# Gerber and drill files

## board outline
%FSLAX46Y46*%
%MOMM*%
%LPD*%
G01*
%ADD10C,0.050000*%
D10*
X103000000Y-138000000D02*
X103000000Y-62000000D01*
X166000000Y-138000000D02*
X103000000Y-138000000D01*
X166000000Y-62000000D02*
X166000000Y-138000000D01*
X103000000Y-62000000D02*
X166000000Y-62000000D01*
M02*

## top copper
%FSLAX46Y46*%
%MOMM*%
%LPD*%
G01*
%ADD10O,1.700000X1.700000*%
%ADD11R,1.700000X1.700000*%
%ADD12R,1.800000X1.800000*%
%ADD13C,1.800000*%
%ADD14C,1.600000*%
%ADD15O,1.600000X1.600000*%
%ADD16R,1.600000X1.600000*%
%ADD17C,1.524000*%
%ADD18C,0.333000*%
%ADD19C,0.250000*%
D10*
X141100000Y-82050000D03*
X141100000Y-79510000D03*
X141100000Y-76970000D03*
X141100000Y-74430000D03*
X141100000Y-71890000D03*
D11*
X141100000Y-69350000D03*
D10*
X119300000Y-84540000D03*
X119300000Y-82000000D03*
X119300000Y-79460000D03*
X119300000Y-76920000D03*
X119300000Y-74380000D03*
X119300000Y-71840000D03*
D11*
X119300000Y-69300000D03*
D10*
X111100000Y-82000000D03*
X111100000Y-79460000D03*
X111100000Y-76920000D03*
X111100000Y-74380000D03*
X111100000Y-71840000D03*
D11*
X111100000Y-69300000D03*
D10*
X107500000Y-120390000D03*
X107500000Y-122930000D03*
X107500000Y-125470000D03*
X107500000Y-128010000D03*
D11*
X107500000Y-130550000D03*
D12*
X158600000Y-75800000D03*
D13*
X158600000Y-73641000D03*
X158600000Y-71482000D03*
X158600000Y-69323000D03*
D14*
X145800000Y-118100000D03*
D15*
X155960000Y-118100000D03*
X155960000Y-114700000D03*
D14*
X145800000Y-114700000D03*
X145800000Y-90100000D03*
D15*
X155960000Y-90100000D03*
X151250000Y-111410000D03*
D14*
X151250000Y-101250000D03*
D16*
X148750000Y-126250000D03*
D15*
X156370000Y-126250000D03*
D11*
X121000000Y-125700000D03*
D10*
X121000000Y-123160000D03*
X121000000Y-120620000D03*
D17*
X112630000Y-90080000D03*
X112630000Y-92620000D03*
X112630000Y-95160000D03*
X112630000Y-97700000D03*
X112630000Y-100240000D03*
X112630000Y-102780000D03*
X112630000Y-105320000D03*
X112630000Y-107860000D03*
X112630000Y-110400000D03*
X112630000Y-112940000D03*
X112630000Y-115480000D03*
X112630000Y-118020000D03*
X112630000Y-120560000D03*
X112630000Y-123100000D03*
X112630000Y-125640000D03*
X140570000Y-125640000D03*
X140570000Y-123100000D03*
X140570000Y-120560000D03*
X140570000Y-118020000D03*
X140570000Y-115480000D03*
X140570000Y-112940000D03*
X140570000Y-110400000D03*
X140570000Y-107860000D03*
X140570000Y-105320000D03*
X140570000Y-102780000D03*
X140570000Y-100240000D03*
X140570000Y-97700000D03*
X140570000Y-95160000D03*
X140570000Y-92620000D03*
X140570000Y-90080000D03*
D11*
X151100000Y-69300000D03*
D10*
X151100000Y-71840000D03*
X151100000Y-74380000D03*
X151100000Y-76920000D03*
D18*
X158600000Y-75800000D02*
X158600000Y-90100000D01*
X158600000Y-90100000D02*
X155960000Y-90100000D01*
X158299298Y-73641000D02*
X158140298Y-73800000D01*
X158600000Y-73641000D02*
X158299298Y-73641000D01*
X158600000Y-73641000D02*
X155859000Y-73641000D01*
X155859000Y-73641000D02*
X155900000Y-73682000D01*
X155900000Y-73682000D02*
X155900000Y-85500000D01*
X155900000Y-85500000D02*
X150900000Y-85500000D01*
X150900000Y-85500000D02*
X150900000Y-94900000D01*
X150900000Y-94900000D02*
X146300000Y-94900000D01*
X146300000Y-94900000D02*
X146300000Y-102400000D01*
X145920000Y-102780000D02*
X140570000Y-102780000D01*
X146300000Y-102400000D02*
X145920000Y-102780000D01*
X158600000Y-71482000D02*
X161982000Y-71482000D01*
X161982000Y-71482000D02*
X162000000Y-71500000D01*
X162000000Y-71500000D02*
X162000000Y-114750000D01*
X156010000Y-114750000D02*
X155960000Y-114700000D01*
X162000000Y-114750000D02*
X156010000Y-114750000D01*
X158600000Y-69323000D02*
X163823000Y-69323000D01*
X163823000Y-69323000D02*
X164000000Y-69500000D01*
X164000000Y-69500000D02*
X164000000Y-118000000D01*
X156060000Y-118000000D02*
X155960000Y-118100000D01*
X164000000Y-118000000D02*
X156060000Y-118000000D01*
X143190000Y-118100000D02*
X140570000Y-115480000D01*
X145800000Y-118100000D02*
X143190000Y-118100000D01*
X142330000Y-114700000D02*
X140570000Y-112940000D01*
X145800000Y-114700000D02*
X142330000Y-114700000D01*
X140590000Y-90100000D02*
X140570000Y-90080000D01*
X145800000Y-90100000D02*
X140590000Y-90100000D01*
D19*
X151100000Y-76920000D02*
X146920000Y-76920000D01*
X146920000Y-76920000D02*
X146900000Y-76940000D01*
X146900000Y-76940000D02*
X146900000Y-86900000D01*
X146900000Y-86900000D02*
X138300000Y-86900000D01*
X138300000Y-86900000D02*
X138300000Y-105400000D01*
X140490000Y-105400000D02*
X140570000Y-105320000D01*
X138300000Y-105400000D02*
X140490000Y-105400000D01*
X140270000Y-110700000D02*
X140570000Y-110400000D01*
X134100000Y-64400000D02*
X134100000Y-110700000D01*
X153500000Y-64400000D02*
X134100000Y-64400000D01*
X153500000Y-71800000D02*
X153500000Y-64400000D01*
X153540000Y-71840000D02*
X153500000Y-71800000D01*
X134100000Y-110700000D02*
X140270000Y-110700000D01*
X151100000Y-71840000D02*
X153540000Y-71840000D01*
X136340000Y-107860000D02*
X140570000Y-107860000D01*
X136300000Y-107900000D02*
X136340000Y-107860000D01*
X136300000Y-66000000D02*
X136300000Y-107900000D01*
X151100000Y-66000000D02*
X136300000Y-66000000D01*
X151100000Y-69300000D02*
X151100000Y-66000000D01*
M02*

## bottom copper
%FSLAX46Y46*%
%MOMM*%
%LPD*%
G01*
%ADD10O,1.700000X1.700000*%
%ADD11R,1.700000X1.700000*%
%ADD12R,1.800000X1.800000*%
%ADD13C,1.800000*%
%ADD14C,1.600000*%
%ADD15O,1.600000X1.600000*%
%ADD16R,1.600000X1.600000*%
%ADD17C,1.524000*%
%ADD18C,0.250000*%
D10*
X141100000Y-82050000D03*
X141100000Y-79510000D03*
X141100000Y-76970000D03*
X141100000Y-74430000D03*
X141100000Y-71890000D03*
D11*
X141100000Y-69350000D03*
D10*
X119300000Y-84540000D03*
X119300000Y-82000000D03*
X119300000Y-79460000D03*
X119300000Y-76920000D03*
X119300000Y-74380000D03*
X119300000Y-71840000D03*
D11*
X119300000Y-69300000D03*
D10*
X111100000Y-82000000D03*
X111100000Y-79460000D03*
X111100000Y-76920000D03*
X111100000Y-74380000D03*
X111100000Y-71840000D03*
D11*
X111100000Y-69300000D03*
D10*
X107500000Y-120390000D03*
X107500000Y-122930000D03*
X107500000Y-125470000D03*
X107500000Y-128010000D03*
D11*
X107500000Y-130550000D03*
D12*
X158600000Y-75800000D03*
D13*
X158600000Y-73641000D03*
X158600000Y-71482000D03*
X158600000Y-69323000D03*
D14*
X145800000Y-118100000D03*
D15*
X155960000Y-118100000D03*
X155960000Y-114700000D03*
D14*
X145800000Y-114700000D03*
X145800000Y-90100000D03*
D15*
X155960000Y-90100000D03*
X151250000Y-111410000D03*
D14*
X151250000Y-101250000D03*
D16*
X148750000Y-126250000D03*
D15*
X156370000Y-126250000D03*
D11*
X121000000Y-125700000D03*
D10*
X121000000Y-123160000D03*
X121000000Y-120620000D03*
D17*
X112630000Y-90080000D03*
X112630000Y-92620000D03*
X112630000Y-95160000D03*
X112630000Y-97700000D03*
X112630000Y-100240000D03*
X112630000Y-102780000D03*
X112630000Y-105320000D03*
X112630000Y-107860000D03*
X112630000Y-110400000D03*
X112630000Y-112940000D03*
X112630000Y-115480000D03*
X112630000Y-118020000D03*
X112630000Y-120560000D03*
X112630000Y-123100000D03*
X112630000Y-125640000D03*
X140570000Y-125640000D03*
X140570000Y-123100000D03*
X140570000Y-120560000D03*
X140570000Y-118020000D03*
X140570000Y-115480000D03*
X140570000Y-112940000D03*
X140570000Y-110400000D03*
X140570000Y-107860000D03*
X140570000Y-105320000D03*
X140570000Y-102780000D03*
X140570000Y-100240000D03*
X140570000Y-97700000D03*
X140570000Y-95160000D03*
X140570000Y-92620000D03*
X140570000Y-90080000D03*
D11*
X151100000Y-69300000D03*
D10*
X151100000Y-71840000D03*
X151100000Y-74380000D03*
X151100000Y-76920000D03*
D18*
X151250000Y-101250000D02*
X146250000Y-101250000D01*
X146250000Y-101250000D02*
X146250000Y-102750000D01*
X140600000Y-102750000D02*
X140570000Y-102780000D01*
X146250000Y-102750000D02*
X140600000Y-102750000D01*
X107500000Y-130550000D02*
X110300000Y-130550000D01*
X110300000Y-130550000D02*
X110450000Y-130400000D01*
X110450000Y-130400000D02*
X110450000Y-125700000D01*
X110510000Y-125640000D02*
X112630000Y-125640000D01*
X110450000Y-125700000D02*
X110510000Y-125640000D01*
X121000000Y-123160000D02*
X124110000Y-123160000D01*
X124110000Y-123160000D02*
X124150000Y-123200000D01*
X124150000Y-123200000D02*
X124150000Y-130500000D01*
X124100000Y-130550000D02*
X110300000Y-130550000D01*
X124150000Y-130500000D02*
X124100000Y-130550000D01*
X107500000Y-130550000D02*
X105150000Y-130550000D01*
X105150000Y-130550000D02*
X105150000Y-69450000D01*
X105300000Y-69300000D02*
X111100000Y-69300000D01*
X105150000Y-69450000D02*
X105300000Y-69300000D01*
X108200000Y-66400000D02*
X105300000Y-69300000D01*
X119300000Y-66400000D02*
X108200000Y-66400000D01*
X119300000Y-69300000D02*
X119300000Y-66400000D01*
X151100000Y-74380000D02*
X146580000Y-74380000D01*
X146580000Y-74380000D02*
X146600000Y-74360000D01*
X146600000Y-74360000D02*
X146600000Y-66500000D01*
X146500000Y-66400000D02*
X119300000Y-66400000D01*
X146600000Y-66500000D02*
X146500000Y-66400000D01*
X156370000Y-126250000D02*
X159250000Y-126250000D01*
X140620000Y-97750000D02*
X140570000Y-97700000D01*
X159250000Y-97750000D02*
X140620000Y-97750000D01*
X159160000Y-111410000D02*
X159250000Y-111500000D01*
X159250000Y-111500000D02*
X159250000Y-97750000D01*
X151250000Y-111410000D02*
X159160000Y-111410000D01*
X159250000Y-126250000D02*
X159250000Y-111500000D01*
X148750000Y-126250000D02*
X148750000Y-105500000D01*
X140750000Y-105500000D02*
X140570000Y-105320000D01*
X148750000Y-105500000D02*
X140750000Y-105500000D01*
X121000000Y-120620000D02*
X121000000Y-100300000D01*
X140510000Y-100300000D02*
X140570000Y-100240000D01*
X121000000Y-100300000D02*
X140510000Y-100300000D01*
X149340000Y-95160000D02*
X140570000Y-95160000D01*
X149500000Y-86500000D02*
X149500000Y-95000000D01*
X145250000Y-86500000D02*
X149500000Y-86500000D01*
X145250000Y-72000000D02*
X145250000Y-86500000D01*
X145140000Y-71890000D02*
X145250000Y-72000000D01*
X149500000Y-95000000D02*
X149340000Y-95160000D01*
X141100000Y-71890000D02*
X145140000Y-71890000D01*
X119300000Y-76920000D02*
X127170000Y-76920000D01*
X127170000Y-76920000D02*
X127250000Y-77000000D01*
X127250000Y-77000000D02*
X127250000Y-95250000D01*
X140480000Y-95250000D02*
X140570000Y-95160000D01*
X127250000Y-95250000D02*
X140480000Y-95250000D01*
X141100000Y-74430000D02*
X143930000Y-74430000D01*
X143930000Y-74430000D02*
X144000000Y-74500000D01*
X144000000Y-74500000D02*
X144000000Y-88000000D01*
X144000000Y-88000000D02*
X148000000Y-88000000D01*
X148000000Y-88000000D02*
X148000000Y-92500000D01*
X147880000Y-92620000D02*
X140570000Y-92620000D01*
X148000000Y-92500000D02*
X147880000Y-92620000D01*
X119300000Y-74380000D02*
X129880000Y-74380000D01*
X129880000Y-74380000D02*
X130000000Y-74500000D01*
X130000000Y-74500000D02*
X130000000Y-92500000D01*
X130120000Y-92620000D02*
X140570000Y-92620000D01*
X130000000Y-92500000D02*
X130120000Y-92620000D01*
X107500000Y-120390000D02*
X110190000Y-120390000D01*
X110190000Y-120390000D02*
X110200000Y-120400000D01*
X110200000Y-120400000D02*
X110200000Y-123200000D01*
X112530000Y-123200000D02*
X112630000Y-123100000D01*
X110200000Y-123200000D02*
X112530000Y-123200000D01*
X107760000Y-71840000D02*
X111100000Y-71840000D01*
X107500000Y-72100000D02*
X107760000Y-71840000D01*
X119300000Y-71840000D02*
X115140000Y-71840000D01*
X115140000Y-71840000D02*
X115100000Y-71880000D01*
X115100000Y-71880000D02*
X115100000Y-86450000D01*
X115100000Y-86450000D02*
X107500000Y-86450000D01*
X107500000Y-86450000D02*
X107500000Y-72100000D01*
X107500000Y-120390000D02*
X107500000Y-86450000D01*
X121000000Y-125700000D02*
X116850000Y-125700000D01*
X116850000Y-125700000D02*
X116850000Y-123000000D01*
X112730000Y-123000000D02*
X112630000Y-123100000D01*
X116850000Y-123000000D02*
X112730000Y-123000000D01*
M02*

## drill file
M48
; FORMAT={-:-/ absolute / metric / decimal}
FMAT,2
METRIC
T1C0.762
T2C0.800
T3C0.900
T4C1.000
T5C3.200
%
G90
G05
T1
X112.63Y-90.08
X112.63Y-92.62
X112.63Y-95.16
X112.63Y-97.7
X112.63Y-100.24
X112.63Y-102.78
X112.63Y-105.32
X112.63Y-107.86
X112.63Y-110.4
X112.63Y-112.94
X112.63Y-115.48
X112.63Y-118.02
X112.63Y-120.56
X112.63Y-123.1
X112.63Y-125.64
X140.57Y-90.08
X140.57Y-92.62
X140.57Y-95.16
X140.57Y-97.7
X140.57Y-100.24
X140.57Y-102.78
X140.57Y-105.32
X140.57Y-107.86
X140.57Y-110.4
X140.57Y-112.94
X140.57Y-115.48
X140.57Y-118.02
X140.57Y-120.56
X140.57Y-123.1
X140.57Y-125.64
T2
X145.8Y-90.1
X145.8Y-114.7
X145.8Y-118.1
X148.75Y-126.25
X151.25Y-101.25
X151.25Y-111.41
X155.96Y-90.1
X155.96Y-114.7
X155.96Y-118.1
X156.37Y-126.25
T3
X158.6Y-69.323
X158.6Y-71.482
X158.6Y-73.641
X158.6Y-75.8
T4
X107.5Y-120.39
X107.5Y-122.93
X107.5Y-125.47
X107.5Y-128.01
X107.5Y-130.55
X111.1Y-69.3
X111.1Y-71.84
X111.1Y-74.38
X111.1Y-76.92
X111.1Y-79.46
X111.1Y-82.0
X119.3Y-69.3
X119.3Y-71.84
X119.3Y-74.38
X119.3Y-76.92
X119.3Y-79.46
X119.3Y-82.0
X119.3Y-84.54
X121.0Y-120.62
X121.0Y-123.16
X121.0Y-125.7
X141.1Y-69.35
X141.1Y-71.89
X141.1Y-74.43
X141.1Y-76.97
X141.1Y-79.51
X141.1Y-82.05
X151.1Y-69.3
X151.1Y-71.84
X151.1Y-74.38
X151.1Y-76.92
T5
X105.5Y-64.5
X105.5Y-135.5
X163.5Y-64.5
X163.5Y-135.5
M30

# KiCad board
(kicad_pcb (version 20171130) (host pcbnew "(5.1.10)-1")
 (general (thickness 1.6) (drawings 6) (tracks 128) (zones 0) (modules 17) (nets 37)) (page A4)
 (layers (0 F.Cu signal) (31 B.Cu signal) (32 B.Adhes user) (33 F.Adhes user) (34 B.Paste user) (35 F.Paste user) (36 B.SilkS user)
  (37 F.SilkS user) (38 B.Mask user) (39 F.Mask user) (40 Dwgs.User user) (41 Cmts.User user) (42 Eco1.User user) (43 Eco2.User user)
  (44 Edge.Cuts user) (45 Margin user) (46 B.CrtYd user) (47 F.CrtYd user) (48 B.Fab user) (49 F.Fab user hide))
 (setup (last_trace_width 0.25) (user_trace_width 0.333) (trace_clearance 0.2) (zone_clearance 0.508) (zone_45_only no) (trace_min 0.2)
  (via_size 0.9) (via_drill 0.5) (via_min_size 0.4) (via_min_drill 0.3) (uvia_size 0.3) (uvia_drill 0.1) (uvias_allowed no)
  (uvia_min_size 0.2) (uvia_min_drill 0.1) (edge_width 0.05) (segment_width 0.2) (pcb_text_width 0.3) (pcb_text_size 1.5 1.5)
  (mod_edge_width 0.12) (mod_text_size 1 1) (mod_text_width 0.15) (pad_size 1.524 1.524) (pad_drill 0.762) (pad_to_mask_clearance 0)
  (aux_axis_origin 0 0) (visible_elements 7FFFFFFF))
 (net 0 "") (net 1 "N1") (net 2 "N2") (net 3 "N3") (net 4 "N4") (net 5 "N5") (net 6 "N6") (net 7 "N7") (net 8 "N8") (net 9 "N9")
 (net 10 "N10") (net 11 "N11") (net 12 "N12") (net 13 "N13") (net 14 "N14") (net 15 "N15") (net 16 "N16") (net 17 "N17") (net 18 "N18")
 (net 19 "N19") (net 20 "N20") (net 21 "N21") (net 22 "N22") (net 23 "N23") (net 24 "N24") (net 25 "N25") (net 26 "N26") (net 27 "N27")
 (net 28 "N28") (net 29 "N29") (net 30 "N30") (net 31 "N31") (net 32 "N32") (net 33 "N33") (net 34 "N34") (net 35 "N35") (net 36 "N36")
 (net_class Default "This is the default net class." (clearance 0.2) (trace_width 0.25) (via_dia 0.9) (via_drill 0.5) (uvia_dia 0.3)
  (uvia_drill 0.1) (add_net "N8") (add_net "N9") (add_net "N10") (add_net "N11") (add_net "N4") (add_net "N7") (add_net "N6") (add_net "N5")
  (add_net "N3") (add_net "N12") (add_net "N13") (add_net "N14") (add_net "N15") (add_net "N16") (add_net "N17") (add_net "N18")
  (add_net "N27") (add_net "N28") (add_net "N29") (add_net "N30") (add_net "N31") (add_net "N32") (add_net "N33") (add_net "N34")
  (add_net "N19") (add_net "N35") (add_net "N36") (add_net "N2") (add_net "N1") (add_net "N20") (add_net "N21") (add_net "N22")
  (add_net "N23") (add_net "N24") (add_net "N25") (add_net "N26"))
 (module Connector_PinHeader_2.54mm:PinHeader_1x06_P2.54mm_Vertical (layer F.Cu) (at 141.1 69.35)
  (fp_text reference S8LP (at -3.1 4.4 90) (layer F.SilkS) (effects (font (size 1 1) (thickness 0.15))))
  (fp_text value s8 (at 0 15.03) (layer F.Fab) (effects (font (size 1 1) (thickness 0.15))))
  (pad 6 thru_hole oval (at 0 12.7) (size 1.7 1.7) (drill 1) (layers *.Cu *.Mask))
  (pad 5 thru_hole oval (at 0 10.16) (size 1.7 1.7) (drill 1) (layers *.Cu *.Mask))
  (pad 4 thru_hole oval (at 0 7.62) (size 1.7 1.7) (drill 1) (layers *.Cu *.Mask))
  (pad 3 thru_hole oval (at 0 5.08) (size 1.7 1.7) (drill 1) (layers *.Cu *.Mask) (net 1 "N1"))
  (pad 2 thru_hole oval (at 0 2.54) (size 1.7 1.7) (drill 1) (layers *.Cu *.Mask) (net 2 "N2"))
  (pad 1 thru_hole rect (at 0 0) (size 1.7 1.7) (drill 1) (layers *.Cu *.Mask)))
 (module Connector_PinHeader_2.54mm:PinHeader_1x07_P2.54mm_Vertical (layer F.Cu) (at 119.3 69.3)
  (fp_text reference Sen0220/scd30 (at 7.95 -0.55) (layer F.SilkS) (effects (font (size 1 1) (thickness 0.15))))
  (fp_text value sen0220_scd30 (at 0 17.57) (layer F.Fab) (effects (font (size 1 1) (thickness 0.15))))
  (pad 7 thru_hole oval (at 0 15.24) (size 1.7 1.7) (drill 1) (layers *.Cu *.Mask))
  (pad 6 thru_hole oval (at 0 12.7) (size 1.7 1.7) (drill 1) (layers *.Cu *.Mask))
  (pad 5 thru_hole oval (at 0 10.16) (size 1.7 1.7) (drill 1) (layers *.Cu *.Mask))
  (pad 4 thru_hole oval (at 0 7.62) (size 1.7 1.7) (drill 1) (layers *.Cu *.Mask) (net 2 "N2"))
  (pad 3 thru_hole oval (at 0 5.08) (size 1.7 1.7) (drill 1) (layers *.Cu *.Mask) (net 1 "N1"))
  (pad 2 thru_hole oval (at 0 2.54) (size 1.7 1.7) (drill 1) (layers *.Cu *.Mask) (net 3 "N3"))
  (pad 1 thru_hole rect (at 0 0) (size 1.7 1.7) (drill 1) (layers *.Cu *.Mask) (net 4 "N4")))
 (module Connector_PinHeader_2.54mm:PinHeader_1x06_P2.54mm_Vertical (layer F.Cu) (at 111.1 69.3)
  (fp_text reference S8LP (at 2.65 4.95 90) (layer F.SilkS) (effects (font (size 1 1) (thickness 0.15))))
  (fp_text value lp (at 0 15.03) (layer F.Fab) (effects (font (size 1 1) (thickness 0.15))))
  (pad 6 thru_hole oval (at 0 12.7) (size 1.7 1.7) (drill 1) (layers *.Cu *.Mask))
  (pad 5 thru_hole oval (at 0 10.16) (size 1.7 1.7) (drill 1) (layers *.Cu *.Mask))
  (pad 4 thru_hole oval (at 0 7.62) (size 1.7 1.7) (drill 1) (layers *.Cu *.Mask))
  (pad 3 thru_hole oval (at 0 5.08) (size 1.7 1.7) (drill 1) (layers *.Cu *.Mask))
  (pad 2 thru_hole oval (at 0 2.54) (size 1.7 1.7) (drill 1) (layers *.Cu *.Mask) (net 3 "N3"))
  (pad 1 thru_hole rect (at 0 0) (size 1.7 1.7) (drill 1) (layers *.Cu *.Mask) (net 4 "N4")))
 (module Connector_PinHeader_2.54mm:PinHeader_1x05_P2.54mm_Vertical (layer F.Cu) (at 107.5 130.55 180)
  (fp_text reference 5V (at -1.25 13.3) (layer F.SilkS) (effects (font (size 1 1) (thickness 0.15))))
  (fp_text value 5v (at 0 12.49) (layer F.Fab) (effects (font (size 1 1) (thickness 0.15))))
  (pad 5 thru_hole oval (at 0 10.16 180) (size 1.7 1.7) (drill 1) (layers *.Cu *.Mask) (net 3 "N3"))
  (pad 4 thru_hole oval (at 0 7.62 180) (size 1.7 1.7) (drill 1) (layers *.Cu *.Mask) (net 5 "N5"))
  (pad 3 thru_hole oval (at 0 5.08 180) (size 1.7 1.7) (drill 1) (layers *.Cu *.Mask) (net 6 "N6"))
  (pad 2 thru_hole oval (at 0 2.54 180) (size 1.7 1.7) (drill 1) (layers *.Cu *.Mask) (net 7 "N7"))
  (pad 1 thru_hole rect (at 0 0 180) (size 1.7 1.7) (drill 1) (layers *.Cu *.Mask) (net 4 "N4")))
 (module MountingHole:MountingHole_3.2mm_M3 (layer F.Cu) (at 105.5 64.5)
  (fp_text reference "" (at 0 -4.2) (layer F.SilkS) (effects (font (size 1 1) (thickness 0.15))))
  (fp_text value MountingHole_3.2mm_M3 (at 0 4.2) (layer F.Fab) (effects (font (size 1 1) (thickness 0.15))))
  (pad 1 np_thru_hole circle (at 0 0) (size 3.2 3.2) (drill 3.2) (layers *.Cu *.Mask)))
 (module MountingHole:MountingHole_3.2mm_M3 (layer F.Cu) (at 105.5 135.5)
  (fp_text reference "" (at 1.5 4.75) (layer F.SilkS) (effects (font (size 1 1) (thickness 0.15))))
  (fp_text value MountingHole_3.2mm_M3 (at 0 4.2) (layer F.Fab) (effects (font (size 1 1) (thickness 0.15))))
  (pad 1 np_thru_hole circle (at 0 0) (size 3.2 3.2) (drill 3.2) (layers *.Cu *.Mask)))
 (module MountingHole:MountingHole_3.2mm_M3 (layer F.Cu) (at 163.5 135.5)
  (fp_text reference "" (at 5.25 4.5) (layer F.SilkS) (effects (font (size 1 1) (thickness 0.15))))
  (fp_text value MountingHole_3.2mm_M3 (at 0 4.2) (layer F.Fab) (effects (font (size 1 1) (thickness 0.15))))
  (pad 1 np_thru_hole circle (at 0 0) (size 3.2 3.2) (drill 3.2) (layers *.Cu *.Mask)))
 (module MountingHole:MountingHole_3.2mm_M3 (layer F.Cu) (at 163.5 64.5)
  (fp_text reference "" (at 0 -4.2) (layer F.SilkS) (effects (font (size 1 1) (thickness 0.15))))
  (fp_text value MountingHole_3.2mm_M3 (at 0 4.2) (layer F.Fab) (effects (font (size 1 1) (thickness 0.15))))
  (pad 1 np_thru_hole circle (at 0 0) (size 3.2 3.2) (drill 3.2) (layers *.Cu *.Mask)))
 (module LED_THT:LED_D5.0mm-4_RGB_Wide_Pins (layer F.Cu) (at 158.6 75.8 90)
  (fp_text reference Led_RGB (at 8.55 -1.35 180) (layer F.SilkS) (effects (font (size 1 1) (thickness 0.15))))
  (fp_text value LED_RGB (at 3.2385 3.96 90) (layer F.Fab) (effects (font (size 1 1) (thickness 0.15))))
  (pad 1 thru_hole rect (at 0 0 90) (size 1.8 1.8) (drill 0.9) (layers *.Cu *.Mask) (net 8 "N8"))
  (pad 2 thru_hole circle (at 2.159 0 90) (size 1.8 1.8) (drill 0.9) (layers *.Cu *.Mask) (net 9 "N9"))
  (pad 3 thru_hole circle (at 4.318 0 90) (size 1.8 1.8) (drill 0.9) (layers *.Cu *.Mask) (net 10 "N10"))
  (pad 4 thru_hole circle (at 6.477 0 90) (size 1.8 1.8) (drill 0.9) (layers *.Cu *.Mask) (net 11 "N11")))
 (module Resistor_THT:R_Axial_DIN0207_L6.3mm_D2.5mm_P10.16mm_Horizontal (layer F.Cu) (at 145.8 118.1)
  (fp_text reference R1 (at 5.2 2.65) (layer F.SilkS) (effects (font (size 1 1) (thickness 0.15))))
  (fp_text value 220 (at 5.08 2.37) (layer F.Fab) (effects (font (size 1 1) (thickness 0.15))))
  (pad 1 thru_hole circle (at 0 0) (size 1.6 1.6) (drill 0.8) (layers *.Cu *.Mask) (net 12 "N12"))
  (pad 2 thru_hole oval (at 10.16 0) (size 1.6 1.6) (drill 0.8) (layers *.Cu *.Mask) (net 11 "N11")))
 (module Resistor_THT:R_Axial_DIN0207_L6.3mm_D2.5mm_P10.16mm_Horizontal (layer F.Cu) (at 145.8 114.7)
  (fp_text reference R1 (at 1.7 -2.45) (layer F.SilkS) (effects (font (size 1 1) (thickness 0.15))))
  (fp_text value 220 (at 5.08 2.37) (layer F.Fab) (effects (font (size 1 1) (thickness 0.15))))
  (pad 2 thru_hole oval (at 10.16 0) (size 1.6 1.6) (drill 0.8) (layers *.Cu *.Mask) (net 10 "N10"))
  (pad 1 thru_hole circle (at 0 0) (size 1.6 1.6) (drill 0.8) (layers *.Cu *.Mask) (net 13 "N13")))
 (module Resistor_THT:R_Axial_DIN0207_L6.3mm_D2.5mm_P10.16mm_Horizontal (layer F.Cu) (at 145.8 90.1)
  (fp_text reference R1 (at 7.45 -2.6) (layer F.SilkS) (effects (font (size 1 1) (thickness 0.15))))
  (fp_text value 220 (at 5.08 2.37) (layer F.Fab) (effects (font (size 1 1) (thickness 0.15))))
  (pad 1 thru_hole circle (at 0 0) (size 1.6 1.6) (drill 0.8) (layers *.Cu *.Mask) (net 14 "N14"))
  (pad 2 thru_hole oval (at 10.16 0) (size 1.6 1.6) (drill 0.8) (layers *.Cu *.Mask) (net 8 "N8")))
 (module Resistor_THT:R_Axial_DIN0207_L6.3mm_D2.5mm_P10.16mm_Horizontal (layer F.Cu) (at 151.25 101.25 270)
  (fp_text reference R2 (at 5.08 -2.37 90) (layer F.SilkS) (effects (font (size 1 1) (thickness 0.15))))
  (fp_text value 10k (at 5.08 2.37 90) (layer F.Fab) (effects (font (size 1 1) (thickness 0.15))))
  (pad 2 thru_hole oval (at 10.16 0 270) (size 1.6 1.6) (drill 0.8) (layers *.Cu *.Mask) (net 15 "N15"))
  (pad 1 thru_hole circle (at 0 0 270) (size 1.6 1.6) (drill 0.8) (layers *.Cu *.Mask) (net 9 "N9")))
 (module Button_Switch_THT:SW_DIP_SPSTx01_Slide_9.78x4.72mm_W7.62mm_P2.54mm (layer F.Cu) (at 148.75 126.25)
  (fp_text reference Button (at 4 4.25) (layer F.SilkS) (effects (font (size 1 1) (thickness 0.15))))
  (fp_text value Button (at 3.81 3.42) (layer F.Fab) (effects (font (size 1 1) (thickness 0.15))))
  (pad 1 thru_hole rect (at 0 0) (size 1.6 1.6) (drill 0.8) (layers *.Cu *.Mask) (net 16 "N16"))
  (pad 2 thru_hole oval (at 7.62 0) (size 1.6 1.6) (drill 0.8) (layers *.Cu *.Mask) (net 15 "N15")))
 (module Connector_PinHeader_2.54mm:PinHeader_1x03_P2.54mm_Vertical (layer F.Cu) (at 121 125.7 180)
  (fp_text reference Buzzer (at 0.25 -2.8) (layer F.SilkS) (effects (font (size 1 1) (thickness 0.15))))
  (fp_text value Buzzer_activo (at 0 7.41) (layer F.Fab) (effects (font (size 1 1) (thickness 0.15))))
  (pad 1 thru_hole rect (at 0 0 180) (size 1.7 1.7) (drill 1) (layers *.Cu *.Mask) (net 3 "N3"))
  (pad 2 thru_hole oval (at 0 2.54 180) (size 1.7 1.7) (drill 1) (layers *.Cu *.Mask) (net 4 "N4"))
  (pad 3 thru_hole oval (at 0 5.08 180) (size 1.7 1.7) (drill 1) (layers *.Cu *.Mask) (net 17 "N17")))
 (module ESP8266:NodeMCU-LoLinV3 (layer F.Cu) (at 126.6 110.4)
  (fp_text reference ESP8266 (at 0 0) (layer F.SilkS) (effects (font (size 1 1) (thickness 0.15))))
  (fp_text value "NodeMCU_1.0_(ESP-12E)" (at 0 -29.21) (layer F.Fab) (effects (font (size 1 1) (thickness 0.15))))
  (pad 1 thru_hole circle (at -13.97 -20.32) (size 1.524 1.524) (drill 0.762) (layers *.Cu *.Mask F.SilkS) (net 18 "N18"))
  (pad 2 thru_hole circle (at -13.97 -17.78) (size 1.524 1.524) (drill 0.762) (layers *.Cu *.Mask F.SilkS) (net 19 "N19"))
  (pad 3 thru_hole circle (at -13.97 -15.24) (size 1.524 1.524) (drill 0.762) (layers *.Cu *.Mask F.SilkS) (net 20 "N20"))
  (pad 4 thru_hole circle (at -13.97 -12.7) (size 1.524 1.524) (drill 0.762) (layers *.Cu *.Mask F.SilkS) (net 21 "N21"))
  (pad 5 thru_hole circle (at -13.97 -10.16) (size 1.524 1.524) (drill 0.762) (layers *.Cu *.Mask F.SilkS) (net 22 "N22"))
  (pad 6 thru_hole circle (at -13.97 -7.62) (size 1.524 1.524) (drill 0.762) (layers *.Cu *.Mask F.SilkS) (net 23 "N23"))
  (pad 7 thru_hole circle (at -13.97 -5.08) (size 1.524 1.524) (drill 0.762) (layers *.Cu *.Mask F.SilkS) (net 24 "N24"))
  (pad 8 thru_hole circle (at -13.97 -2.54) (size 1.524 1.524) (drill 0.762) (layers *.Cu *.Mask F.SilkS) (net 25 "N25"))
  (pad 9 thru_hole circle (at -13.97 0) (size 1.524 1.524) (drill 0.762) (layers *.Cu *.Mask F.SilkS) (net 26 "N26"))
  (pad 10 thru_hole circle (at -13.97 2.54) (size 1.524 1.524) (drill 0.762) (layers *.Cu *.Mask F.SilkS) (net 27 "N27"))
  (pad 11 thru_hole circle (at -13.97 5.08) (size 1.524 1.524) (drill 0.762) (layers *.Cu *.Mask F.SilkS) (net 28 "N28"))
  (pad 12 thru_hole circle (at -13.97 7.62) (size 1.524 1.524) (drill 0.762) (layers *.Cu *.Mask F.SilkS) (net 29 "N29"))
  (pad 13 thru_hole circle (at -13.97 10.16) (size 1.524 1.524) (drill 0.762) (layers *.Cu *.Mask F.SilkS) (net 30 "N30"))
  (pad 14 thru_hole circle (at -13.97 12.7) (size 1.524 1.524) (drill 0.762) (layers *.Cu *.Mask F.SilkS) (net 3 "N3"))
  (pad 15 thru_hole circle (at -13.97 15.24) (size 1.524 1.524) (drill 0.762) (layers *.Cu *.Mask F.SilkS) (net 4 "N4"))
  (pad 16 thru_hole circle (at 13.97 15.24) (size 1.524 1.524) (drill 0.762) (layers *.Cu *.Mask F.SilkS) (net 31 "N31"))
  (pad 17 thru_hole circle (at 13.97 12.7) (size 1.524 1.524) (drill 0.762) (layers *.Cu *.Mask F.SilkS) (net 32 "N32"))
  (pad 18 thru_hole circle (at 13.97 10.16) (size 1.524 1.524) (drill 0.762) (layers *.Cu *.Mask F.SilkS) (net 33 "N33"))
  (pad 19 thru_hole circle (at 13.97 7.62) (size 1.524 1.524) (drill 0.762) (layers *.Cu *.Mask F.SilkS) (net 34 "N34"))
  (pad 20 thru_hole circle (at 13.97 5.08) (size 1.524 1.524) (drill 0.762) (layers *.Cu *.Mask F.SilkS) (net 12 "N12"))
  (pad 21 thru_hole circle (at 13.97 2.54) (size 1.524 1.524) (drill 0.762) (layers *.Cu *.Mask F.SilkS) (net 13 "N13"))
  (pad 22 thru_hole circle (at 13.97 0) (size 1.524 1.524) (drill 0.762) (layers *.Cu *.Mask F.SilkS) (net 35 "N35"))
  (pad 23 thru_hole circle (at 13.97 -2.54) (size 1.524 1.524) (drill 0.762) (layers *.Cu *.Mask F.SilkS) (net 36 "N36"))
  (pad 24 thru_hole circle (at 13.97 -5.08) (size 1.524 1.524) (drill 0.762) (layers *.Cu *.Mask F.SilkS) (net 16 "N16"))
  (pad 25 thru_hole circle (at 13.97 -7.62) (size 1.524 1.524) (drill 0.762) (layers *.Cu *.Mask F.SilkS) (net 9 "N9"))
  (pad 26 thru_hole circle (at 13.97 -10.16) (size 1.524 1.524) (drill 0.762) (layers *.Cu *.Mask F.SilkS) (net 17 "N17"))
  (pad 27 thru_hole circle (at 13.97 -12.7) (size 1.524 1.524) (drill 0.762) (layers *.Cu *.Mask F.SilkS) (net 15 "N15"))
  (pad 28 thru_hole circle (at 13.97 -15.24) (size 1.524 1.524) (drill 0.762) (layers *.Cu *.Mask F.SilkS) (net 2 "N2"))
  (pad 29 thru_hole circle (at 13.97 -17.78) (size 1.524 1.524) (drill 0.762) (layers *.Cu *.Mask F.SilkS) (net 1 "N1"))
  (pad 30 thru_hole circle (at 13.97 -20.32) (size 1.524 1.524) (drill 0.762) (layers *.Cu *.Mask F.SilkS) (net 14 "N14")))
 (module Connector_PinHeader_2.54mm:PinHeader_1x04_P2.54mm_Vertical (layer F.Cu) (at 151.1 69.3)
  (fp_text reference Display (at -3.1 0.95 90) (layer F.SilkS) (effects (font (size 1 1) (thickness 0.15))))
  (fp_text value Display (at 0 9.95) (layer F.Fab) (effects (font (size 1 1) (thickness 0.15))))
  (pad 1 thru_hole rect (at 0 0) (size 1.7 1.7) (drill 1) (layers *.Cu *.Mask) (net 36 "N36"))
  (pad 2 thru_hole oval (at 0 2.54) (size 1.7 1.7) (drill 1) (layers *.Cu *.Mask) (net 35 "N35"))
  (pad 3 thru_hole oval (at 0 5.08) (size 1.7 1.7) (drill 1) (layers *.Cu *.Mask) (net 4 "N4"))
  (pad 4 thru_hole oval (at 0 7.62) (size 1.7 1.7) (drill 1) (layers *.Cu *.Mask) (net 16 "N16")))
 (gr_line (start 103 138) (end 103 62) (layer Edge.Cuts) (width 0.05))
 (gr_line (start 166 138) (end 103 138) (layer Edge.Cuts) (width 0.05))
 (gr_line (start 166 62) (end 166 138) (layer Edge.Cuts) (width 0.05))
 (gr_line (start 103 62) (end 166 62) (layer Edge.Cuts) (width 0.05))
 (segment (start 158.6 75.8) (end 158.6 90.1) (width 0.333) (layer F.Cu) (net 8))
 (segment (start 158.6 90.1) (end 155.96 90.1) (width 0.333) (layer F.Cu) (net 8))
 (segment (start 158.299298 73.641) (end 158.140298 73.8) (width 0.333) (layer F.Cu) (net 9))
 (segment (start 158.6 73.641) (end 158.299298 73.641) (width 0.333) (layer F.Cu) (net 9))
 (segment (start 158.6 73.641) (end 155.859 73.641) (width 0.333) (layer F.Cu) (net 9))
 (segment (start 155.859 73.641) (end 155.9 73.682) (width 0.333) (layer F.Cu) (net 9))
 (segment (start 155.9 73.682) (end 155.9 85.5) (width 0.333) (layer F.Cu) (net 9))
 (segment (start 155.9 85.5) (end 150.9 85.5) (width 0.333) (layer F.Cu) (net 9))
 (segment (start 150.9 85.5) (end 150.9 94.9) (width 0.333) (layer F.Cu) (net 9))
 (segment (start 150.9 94.9) (end 146.3 94.9) (width 0.333) (layer F.Cu) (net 9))
 (segment (start 146.3 94.9) (end 146.3 102.4) (width 0.333) (layer F.Cu) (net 9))
 (segment (start 145.92 102.78) (end 140.57 102.78) (width 0.333) (layer F.Cu) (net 9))
 (segment (start 146.3 102.4) (end 145.92 102.78) (width 0.333) (layer F.Cu) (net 9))
 (segment (start 151.25 101.25) (end 146.25 101.25) (width 0.25) (layer B.Cu) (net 9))
 (segment (start 146.25 101.25) (end 146.25 102.75) (width 0.25) (layer B.Cu) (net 9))
 (segment (start 140.6 102.75) (end 140.57 102.78) (width 0.25) (layer B.Cu) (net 9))
 (segment (start 146.25 102.75) (end 140.6 102.75) (width 0.25) (layer B.Cu) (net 9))
 (segment (start 158.6 71.482) (end 161.982 71.482) (width 0.333) (layer F.Cu) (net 10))
 (segment (start 161.982 71.482) (end 162 71.5) (width 0.333) (layer F.Cu) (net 10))
 (segment (start 162 71.5) (end 162 114.75) (width 0.333) (layer F.Cu) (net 10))
 (segment (start 156.01 114.75) (end 155.96 114.7) (width 0.333) (layer F.Cu) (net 10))
 (segment (start 162 114.75) (end 156.01 114.75) (width 0.333) (layer F.Cu) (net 10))
 (segment (start 158.6 69.323) (end 163.823 69.323) (width 0.333) (layer F.Cu) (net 11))
 (segment (start 163.823 69.323) (end 164 69.5) (width 0.333) (layer F.Cu) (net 11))
 (segment (start 164 69.5) (end 164 118) (width 0.333) (layer F.Cu) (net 11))
 (segment (start 156.06 118) (end 155.96 118.1) (width 0.333) (layer F.Cu) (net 11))
 (segment (start 164 118) (end 156.06 118) (width 0.333) (layer F.Cu) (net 11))
 (segment (start 107.5 130.55) (end 110.3 130.55) (width 0.25) (layer B.Cu) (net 4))
 (segment (start 110.3 130.55) (end 110.45 130.4) (width 0.25) (layer B.Cu) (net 4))
 (segment (start 110.45 130.4) (end 110.45 125.7) (width 0.25) (layer B.Cu) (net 4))
 (segment (start 110.51 125.64) (end 112.63 125.64) (width 0.25) (layer B.Cu) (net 4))
 (segment (start 110.45 125.7) (end 110.51 125.64) (width 0.25) (layer B.Cu) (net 4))
 (segment (start 121 123.16) (end 124.11 123.16) (width 0.25) (layer B.Cu) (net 4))
 (segment (start 124.11 123.16) (end 124.15 123.2) (width 0.25) (layer B.Cu) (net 4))
 (segment (start 124.15 123.2) (end 124.15 130.5) (width 0.25) (layer B.Cu) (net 4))
 (segment (start 124.1 130.55) (end 110.3 130.55) (width 0.25) (layer B.Cu) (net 4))
 (segment (start 124.15 130.5) (end 124.1 130.55) (width 0.25) (layer B.Cu) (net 4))
 (segment (start 107.5 130.55) (end 105.15 130.55) (width 0.25) (layer B.Cu) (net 4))
 (segment (start 105.15 130.55) (end 105.15 69.45) (width 0.25) (layer B.Cu) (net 4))
 (segment (start 105.3 69.3) (end 111.1 69.3) (width 0.25) (layer B.Cu) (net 4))
 (segment (start 105.15 69.45) (end 105.3 69.3) (width 0.25) (layer B.Cu) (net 4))
 (segment (start 108.2 66.4) (end 105.3 69.3) (width 0.25) (layer B.Cu) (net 4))
 (segment (start 119.3 66.4) (end 108.2 66.4) (width 0.25) (layer B.Cu) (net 4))
 (segment (start 119.3 69.3) (end 119.3 66.4) (width 0.25) (layer B.Cu) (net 4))
 (segment (start 151.1 74.38) (end 146.58 74.38) (width 0.25) (layer B.Cu) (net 4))
 (segment (start 146.58 74.38) (end 146.6 74.36) (width 0.25) (layer B.Cu) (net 4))
 (segment (start 146.6 74.36) (end 146.6 66.5) (width 0.25) (layer B.Cu) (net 4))
 (segment (start 146.5 66.4) (end 119.3 66.4) (width 0.25) (layer B.Cu) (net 4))
 (segment (start 146.6 66.5) (end 146.5 66.4) (width 0.25) (layer B.Cu) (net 4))
 (segment (start 143.19 118.1) (end 140.57 115.48) (width 0.333) (layer F.Cu) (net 12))
 (segment (start 145.8 118.1) (end 143.19 118.1) (width 0.333) (layer F.Cu) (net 12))
 (segment (start 142.33 114.7) (end 140.57 112.94) (width 0.333) (layer F.Cu) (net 13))
 (segment (start 145.8 114.7) (end 142.33 114.7) (width 0.333) (layer F.Cu) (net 13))
 (segment (start 140.59 90.1) (end 140.57 90.08) (width 0.333) (layer F.Cu) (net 14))
 (segment (start 145.8 90.1) (end 140.59 90.1) (width 0.333) (layer F.Cu) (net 14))
 (segment (start 156.37 126.25) (end 159.25 126.25) (width 0.25) (layer B.Cu) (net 15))
 (segment (start 140.62 97.75) (end 140.57 97.7) (width 0.25) (layer B.Cu) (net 15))
 (segment (start 159.25 97.75) (end 140.62 97.75) (width 0.25) (layer B.Cu) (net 15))
 (segment (start 159.16 111.41) (end 159.25 111.5) (width 0.25) (layer B.Cu) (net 15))
 (segment (start 159.25 111.5) (end 159.25 97.75) (width 0.25) (layer B.Cu) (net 15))
 (segment (start 151.25 111.41) (end 159.16 111.41) (width 0.25) (layer B.Cu) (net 15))
 (segment (start 159.25 126.25) (end 159.25 111.5) (width 0.25) (layer B.Cu) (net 15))
 (segment (start 151.1 76.92) (end 146.92 76.92) (width 0.25) (layer F.Cu) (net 16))
 (segment (start 146.92 76.92) (end 146.9 76.94) (width 0.25) (layer F.Cu) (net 16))
 (segment (start 146.9 76.94) (end 146.9 86.9) (width 0.25) (layer F.Cu) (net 16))
 (segment (start 146.9 86.9) (end 138.3 86.9) (width 0.25) (layer F.Cu) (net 16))
 (segment (start 138.3 86.9) (end 138.3 105.4) (width 0.25) (layer F.Cu) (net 16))
 (segment (start 140.49 105.4) (end 140.57 105.32) (width 0.25) (layer F.Cu) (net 16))
 (segment (start 138.3 105.4) (end 140.49 105.4) (width 0.25) (layer F.Cu) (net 16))
 (segment (start 148.75 126.25) (end 148.75 105.5) (width 0.25) (layer B.Cu) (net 16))
 (segment (start 140.75 105.5) (end 140.57 105.32) (width 0.25) (layer B.Cu) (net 16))
 (segment (start 148.75 105.5) (end 140.75 105.5) (width 0.25) (layer B.Cu) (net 16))
 (segment (start 121 120.62) (end 121 100.3) (width 0.25) (layer B.Cu) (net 17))
 (segment (start 140.51 100.3) (end 140.57 100.24) (width 0.25) (layer B.Cu) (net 17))
 (segment (start 121 100.3) (end 140.51 100.3) (width 0.25) (layer B.Cu) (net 17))
 (segment (start 140.27 110.7) (end 140.57 110.4) (width 0.25) (layer F.Cu) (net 35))
 (segment (start 134.1 64.4) (end 134.1 110.7) (width 0.25) (layer F.Cu) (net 35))
 (segment (start 153.5 64.4) (end 134.1 64.4) (width 0.25) (layer F.Cu) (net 35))
 (segment (start 153.5 71.8) (end 153.5 64.4) (width 0.25) (layer F.Cu) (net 35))
 (segment (start 153.54 71.84) (end 153.5 71.8) (width 0.25) (layer F.Cu) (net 35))
 (segment (start 134.1 110.7) (end 140.27 110.7) (width 0.25) (layer F.Cu) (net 35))
 (segment (start 151.1 71.84) (end 153.54 71.84) (width 0.25) (layer F.Cu) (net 35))
 (segment (start 136.34 107.86) (end 140.57 107.86) (width 0.25) (layer F.Cu) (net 36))
 (segment (start 136.3 107.9) (end 136.34 107.86) (width 0.25) (layer F.Cu) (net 36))
 (segment (start 136.3 66) (end 136.3 107.9) (width 0.25) (layer F.Cu) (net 36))
 (segment (start 151.1 66) (end 136.3 66) (width 0.25) (layer F.Cu) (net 36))
 (segment (start 151.1 69.3) (end 151.1 66) (width 0.25) (layer F.Cu) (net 36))
 (segment (start 149.34 95.16) (end 140.57 95.16) (width 0.25) (layer B.Cu) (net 2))
 (segment (start 149.5 86.5) (end 149.5 95) (width 0.25) (layer B.Cu) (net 2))
 (segment (start 145.25 86.5) (end 149.5 86.5) (width 0.25) (layer B.Cu) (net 2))
 (segment (start 145.25 72) (end 145.25 86.5) (width 0.25) (layer B.Cu) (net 2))
 (segment (start 145.14 71.89) (end 145.25 72) (width 0.25) (layer B.Cu) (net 2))
 (segment (start 149.5 95) (end 149.34 95.16) (width 0.25) (layer B.Cu) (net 2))
 (segment (start 141.1 71.89) (end 145.14 71.89) (width 0.25) (layer B.Cu) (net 2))
 (segment (start 119.3 76.92) (end 127.17 76.92) (width 0.25) (layer B.Cu) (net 2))
 (segment (start 127.17 76.92) (end 127.25 77) (width 0.25) (layer B.Cu) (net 2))
 (segment (start 127.25 77) (end 127.25 95.25) (width 0.25) (layer B.Cu) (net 2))
 (segment (start 140.48 95.25) (end 140.57 95.16) (width 0.25) (layer B.Cu) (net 2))
 (segment (start 127.25 95.25) (end 140.48 95.25) (width 0.25) (layer B.Cu) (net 2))
 (segment (start 141.1 74.43) (end 143.93 74.43) (width 0.25) (layer B.Cu) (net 1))
 (segment (start 143.93 74.43) (end 144 74.5) (width 0.25) (layer B.Cu) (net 1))
 (segment (start 144 74.5) (end 144 88) (width 0.25) (layer B.Cu) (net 1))
 (segment (start 144 88) (end 148 88) (width 0.25) (layer B.Cu) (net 1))
 (segment (start 148 88) (end 148 92.5) (width 0.25) (layer B.Cu) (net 1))
 (segment (start 147.88 92.62) (end 140.57 92.62) (width 0.25) (layer B.Cu) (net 1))
 (segment (start 148 92.5) (end 147.88 92.62) (width 0.25) (layer B.Cu) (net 1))
 (segment (start 119.3 74.38) (end 129.88 74.38) (width 0.25) (layer B.Cu) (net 1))
 (segment (start 129.88 74.38) (end 130 74.5) (width 0.25) (layer B.Cu) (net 1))
 (segment (start 130 74.5) (end 130 92.5) (width 0.25) (layer B.Cu) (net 1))
 (segment (start 130.12 92.62) (end 140.57 92.62) (width 0.25) (layer B.Cu) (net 1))
 (segment (start 130 92.5) (end 130.12 92.62) (width 0.25) (layer B.Cu) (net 1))
 (segment (start 107.5 120.39) (end 110.19 120.39) (width 0.25) (layer B.Cu) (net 3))
 (segment (start 110.19 120.39) (end 110.2 120.4) (width 0.25) (layer B.Cu) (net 3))
 (segment (start 110.2 120.4) (end 110.2 123.2) (width 0.25) (layer B.Cu) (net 3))
 (segment (start 112.53 123.2) (end 112.63 123.1) (width 0.25) (layer B.Cu) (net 3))
 (segment (start 110.2 123.2) (end 112.53 123.2) (width 0.25) (layer B.Cu) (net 3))
 (segment (start 107.76 71.84) (end 111.1 71.84) (width 0.25) (layer B.Cu) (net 3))
 (segment (start 107.5 72.1) (end 107.76 71.84) (width 0.25) (layer B.Cu) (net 3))
 (segment (start 119.3 71.84) (end 115.14 71.84) (width 0.25) (layer B.Cu) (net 3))
 (segment (start 115.14 71.84) (end 115.1 71.88) (width 0.25) (layer B.Cu) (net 3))
 (segment (start 115.1 71.88) (end 115.1 86.45) (width 0.25) (layer B.Cu) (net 3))
 (segment (start 115.1 86.45) (end 107.5 86.45) (width 0.25) (layer B.Cu) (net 3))
 (segment (start 107.5 86.45) (end 107.5 72.1) (width 0.25) (layer B.Cu) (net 3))
 (segment (start 107.5 120.39) (end 107.5 86.45) (width 0.25) (layer B.Cu) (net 3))
 (segment (start 121 125.7) (end 116.85 125.7) (width 0.25) (layer B.Cu) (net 3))
 (segment (start 116.85 125.7) (end 116.85 123) (width 0.25) (layer B.Cu) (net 3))
 (segment (start 112.73 123) (end 112.63 123.1) (width 0.25) (layer B.Cu) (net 3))
 (segment (start 116.85 123) (end 112.73 123) (width 0.25) (layer B.Cu) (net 3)))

